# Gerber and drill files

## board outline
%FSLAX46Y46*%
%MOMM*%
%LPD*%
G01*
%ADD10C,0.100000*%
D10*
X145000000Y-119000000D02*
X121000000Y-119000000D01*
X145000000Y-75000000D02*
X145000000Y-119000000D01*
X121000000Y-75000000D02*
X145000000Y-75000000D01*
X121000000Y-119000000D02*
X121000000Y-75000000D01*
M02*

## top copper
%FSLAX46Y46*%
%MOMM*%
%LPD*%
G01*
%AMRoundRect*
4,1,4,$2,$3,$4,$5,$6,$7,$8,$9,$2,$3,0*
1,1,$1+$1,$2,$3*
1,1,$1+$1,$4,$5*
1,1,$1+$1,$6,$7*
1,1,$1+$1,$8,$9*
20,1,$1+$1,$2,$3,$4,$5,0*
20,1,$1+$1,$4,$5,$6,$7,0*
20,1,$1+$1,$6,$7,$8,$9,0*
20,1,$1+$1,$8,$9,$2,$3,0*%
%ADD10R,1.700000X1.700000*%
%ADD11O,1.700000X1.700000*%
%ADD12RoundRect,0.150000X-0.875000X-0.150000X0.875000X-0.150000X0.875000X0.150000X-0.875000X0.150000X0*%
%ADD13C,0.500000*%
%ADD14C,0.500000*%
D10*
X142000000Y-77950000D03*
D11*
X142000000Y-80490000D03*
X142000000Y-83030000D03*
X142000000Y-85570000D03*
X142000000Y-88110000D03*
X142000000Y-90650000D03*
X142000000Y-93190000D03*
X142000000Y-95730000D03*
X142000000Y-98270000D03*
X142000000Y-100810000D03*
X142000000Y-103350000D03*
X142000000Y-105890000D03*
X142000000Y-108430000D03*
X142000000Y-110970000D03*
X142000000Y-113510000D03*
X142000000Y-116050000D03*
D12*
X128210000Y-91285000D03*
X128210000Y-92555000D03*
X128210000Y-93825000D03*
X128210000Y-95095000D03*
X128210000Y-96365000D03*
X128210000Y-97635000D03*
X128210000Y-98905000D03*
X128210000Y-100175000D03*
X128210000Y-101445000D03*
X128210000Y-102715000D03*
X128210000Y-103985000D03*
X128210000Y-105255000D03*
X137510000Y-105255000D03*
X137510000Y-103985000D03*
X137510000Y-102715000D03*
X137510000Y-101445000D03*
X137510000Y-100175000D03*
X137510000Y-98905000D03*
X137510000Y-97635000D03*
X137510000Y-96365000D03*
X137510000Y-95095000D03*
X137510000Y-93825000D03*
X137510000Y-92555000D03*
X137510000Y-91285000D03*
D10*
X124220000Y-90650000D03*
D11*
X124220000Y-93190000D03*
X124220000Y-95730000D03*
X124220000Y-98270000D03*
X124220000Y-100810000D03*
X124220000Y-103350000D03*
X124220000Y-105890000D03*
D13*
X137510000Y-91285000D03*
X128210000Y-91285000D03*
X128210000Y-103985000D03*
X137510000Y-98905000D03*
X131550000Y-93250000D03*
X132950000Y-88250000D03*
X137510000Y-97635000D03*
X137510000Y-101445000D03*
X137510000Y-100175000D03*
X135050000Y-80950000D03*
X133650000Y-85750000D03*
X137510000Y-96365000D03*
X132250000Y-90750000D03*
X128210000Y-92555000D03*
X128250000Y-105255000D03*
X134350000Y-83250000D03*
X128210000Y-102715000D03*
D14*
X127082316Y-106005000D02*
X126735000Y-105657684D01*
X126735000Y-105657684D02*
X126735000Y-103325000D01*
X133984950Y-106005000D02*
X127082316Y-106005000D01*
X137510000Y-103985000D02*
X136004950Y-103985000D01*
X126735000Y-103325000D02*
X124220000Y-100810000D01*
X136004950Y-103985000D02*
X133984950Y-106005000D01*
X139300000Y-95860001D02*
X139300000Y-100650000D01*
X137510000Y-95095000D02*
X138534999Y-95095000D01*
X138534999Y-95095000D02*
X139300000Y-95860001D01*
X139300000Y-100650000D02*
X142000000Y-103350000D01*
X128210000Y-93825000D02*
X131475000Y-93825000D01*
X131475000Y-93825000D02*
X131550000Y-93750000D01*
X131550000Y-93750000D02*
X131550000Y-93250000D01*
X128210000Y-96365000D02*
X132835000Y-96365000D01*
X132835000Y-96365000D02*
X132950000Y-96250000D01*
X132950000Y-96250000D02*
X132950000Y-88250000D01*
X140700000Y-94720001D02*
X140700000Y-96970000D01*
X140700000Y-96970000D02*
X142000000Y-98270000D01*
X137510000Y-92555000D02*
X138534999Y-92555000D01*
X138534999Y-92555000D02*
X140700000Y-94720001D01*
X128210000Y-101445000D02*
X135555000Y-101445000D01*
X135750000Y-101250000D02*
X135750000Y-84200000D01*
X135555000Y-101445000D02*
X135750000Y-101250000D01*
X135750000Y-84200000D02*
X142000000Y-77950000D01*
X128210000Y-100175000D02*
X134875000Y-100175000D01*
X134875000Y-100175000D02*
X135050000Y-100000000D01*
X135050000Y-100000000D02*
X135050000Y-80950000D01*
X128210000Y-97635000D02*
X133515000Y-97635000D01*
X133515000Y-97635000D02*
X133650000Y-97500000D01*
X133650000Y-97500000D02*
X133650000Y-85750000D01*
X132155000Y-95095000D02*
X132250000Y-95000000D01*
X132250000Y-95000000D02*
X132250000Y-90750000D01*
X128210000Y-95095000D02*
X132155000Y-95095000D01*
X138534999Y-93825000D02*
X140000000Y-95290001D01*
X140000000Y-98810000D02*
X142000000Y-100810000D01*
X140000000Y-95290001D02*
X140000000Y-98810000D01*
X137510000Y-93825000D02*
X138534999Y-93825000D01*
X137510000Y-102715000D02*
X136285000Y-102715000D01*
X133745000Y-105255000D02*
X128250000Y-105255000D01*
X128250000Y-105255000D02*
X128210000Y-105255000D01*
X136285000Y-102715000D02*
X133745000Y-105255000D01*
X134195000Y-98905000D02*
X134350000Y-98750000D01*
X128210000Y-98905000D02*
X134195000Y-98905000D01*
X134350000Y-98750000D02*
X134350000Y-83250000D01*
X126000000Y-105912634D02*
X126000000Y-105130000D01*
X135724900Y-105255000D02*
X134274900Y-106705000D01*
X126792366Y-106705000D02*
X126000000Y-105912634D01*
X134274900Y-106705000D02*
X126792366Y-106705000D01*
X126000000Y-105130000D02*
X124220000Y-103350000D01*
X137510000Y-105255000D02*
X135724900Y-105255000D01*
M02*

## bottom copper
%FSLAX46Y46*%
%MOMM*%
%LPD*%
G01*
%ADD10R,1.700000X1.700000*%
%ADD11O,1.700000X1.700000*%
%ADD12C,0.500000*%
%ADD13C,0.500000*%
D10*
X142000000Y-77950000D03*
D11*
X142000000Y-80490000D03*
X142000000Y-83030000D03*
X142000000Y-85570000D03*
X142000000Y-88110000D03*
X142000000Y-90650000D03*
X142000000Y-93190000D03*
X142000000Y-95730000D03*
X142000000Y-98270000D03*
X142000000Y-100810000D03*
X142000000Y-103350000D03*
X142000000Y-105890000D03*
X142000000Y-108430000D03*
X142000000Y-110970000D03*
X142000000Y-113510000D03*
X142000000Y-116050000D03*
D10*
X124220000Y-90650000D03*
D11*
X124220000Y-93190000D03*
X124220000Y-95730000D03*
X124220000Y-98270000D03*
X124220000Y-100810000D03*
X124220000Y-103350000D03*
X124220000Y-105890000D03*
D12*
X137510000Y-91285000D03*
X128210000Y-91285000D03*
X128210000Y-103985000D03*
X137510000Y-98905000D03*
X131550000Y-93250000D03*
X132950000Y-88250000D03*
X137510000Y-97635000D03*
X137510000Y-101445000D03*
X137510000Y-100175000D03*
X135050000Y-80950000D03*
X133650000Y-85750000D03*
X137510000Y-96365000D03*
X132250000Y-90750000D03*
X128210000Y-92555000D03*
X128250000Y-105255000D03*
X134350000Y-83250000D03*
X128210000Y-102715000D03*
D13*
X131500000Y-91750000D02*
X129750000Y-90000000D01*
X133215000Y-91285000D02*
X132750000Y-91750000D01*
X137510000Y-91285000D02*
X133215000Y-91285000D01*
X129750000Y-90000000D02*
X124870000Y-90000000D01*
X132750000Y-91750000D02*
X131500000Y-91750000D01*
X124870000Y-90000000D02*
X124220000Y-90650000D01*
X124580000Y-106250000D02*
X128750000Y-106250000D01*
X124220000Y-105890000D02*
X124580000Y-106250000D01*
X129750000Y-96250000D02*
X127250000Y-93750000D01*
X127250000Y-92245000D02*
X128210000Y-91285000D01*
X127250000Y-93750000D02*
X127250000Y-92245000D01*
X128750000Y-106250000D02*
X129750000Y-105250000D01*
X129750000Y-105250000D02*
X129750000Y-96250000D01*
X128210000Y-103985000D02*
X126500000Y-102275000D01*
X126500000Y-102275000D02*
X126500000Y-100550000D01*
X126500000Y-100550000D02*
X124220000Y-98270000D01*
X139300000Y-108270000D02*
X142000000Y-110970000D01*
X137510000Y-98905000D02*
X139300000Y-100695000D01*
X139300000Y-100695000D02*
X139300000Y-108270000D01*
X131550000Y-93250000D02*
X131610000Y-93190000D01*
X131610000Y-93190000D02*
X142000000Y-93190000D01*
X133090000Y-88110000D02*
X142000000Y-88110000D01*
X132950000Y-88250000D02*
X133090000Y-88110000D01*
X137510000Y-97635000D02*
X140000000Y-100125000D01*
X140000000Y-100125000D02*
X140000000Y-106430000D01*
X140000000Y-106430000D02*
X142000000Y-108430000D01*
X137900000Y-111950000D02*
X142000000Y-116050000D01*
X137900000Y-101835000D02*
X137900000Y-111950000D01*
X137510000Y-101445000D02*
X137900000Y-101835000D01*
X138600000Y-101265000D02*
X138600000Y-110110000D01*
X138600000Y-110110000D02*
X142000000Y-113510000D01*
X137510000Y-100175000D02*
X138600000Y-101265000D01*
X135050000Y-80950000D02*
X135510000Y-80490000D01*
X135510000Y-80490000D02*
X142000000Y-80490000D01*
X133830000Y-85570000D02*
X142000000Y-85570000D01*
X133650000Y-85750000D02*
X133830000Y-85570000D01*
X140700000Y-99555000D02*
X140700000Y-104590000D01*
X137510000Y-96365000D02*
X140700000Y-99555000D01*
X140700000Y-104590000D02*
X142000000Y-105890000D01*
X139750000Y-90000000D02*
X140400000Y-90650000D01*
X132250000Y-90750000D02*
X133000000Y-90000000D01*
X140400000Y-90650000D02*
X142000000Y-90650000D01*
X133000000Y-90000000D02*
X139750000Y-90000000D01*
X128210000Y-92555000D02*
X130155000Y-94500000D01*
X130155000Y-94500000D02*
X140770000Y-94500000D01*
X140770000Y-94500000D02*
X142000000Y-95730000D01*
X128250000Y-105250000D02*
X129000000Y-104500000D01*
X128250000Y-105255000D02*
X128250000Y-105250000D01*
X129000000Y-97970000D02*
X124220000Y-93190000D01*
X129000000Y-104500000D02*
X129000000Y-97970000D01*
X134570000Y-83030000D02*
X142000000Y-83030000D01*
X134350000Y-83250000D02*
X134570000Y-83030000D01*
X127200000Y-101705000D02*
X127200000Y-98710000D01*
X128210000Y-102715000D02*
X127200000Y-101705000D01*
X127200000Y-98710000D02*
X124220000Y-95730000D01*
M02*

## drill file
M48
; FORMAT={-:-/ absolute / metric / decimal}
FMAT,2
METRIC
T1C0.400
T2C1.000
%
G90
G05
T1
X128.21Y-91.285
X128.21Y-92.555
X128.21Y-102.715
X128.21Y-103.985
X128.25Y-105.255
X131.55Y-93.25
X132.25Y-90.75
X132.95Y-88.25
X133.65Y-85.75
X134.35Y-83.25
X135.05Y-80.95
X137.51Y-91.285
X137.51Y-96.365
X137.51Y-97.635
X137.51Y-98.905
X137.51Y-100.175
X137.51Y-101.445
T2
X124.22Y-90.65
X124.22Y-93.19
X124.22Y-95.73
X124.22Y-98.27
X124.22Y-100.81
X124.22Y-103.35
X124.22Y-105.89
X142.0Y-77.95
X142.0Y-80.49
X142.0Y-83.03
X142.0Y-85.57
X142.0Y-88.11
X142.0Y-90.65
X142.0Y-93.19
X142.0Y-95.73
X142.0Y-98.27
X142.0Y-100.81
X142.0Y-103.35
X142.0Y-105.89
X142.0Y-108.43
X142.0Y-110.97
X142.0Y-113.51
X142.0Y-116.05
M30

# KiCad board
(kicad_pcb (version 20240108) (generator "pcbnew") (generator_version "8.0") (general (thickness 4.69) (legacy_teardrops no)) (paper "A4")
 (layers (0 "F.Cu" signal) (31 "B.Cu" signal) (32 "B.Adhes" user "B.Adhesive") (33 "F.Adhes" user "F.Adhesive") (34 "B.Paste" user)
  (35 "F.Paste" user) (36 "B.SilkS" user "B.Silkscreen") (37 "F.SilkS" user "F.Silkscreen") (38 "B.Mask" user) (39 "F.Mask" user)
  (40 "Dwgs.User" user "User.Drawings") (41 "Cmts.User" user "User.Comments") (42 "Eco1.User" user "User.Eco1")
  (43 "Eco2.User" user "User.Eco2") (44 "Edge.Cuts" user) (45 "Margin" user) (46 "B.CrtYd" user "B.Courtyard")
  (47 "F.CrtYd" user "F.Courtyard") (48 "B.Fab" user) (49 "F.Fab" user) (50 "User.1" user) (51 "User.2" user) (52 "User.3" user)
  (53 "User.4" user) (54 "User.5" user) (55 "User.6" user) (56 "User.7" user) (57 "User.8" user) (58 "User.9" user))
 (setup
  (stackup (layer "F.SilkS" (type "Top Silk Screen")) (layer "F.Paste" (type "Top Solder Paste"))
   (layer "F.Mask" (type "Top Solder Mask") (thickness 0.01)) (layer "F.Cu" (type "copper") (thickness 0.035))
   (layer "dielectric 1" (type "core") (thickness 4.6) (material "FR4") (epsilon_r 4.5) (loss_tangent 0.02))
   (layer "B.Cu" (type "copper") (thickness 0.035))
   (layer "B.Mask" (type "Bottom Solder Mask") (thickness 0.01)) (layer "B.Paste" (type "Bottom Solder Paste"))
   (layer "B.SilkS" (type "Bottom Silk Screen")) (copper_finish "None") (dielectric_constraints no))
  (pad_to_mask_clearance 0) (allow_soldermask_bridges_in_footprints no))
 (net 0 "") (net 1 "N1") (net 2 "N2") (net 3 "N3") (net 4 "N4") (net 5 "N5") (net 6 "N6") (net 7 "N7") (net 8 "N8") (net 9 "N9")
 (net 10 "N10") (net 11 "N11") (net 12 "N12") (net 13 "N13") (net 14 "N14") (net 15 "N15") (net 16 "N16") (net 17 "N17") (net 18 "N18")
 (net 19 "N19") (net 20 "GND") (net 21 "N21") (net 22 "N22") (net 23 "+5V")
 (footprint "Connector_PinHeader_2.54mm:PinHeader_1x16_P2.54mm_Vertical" (layer "F.Cu") (at 142 77.95)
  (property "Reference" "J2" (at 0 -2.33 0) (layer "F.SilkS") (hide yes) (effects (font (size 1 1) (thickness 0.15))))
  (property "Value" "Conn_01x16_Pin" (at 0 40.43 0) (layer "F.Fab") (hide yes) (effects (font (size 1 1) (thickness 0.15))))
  (pad "1" thru_hole rect (at 0 0) (size 1.7 1.7) (drill 1) (layers "*.Cu" "*.Mask") (remove_unused_layers no) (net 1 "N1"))
  (pad "2" thru_hole oval (at 0 2.54) (size 1.7 1.7) (drill 1) (layers "*.Cu" "*.Mask") (remove_unused_layers no) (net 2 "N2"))
  (pad "3" thru_hole oval (at 0 5.08) (size 1.7 1.7) (drill 1) (layers "*.Cu" "*.Mask") (remove_unused_layers no) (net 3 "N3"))
  (pad "4" thru_hole oval (at 0 7.62) (size 1.7 1.7) (drill 1) (layers "*.Cu" "*.Mask") (remove_unused_layers no) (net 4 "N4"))
  (pad "5" thru_hole oval (at 0 10.16) (size 1.7 1.7) (drill 1) (layers "*.Cu" "*.Mask") (remove_unused_layers no) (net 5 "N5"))
  (pad "6" thru_hole oval (at 0 12.7) (size 1.7 1.7) (drill 1) (layers "*.Cu" "*.Mask") (remove_unused_layers no) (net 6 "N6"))
  (pad "7" thru_hole oval (at 0 15.24) (size 1.7 1.7) (drill 1) (layers "*.Cu" "*.Mask") (remove_unused_layers no) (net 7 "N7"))
  (pad "8" thru_hole oval (at 0 17.78) (size 1.7 1.7) (drill 1) (layers "*.Cu" "*.Mask") (remove_unused_layers no) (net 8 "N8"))
  (pad "9" thru_hole oval (at 0 20.32) (size 1.7 1.7) (drill 1) (layers "*.Cu" "*.Mask") (remove_unused_layers no) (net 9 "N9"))
  (pad "10" thru_hole oval (at 0 22.86) (size 1.7 1.7) (drill 1) (layers "*.Cu" "*.Mask") (remove_unused_layers no) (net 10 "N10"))
  (pad "11" thru_hole oval (at 0 25.4) (size 1.7 1.7) (drill 1) (layers "*.Cu" "*.Mask") (remove_unused_layers no) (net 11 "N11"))
  (pad "12" thru_hole oval (at 0 27.94) (size 1.7 1.7) (drill 1) (layers "*.Cu" "*.Mask") (remove_unused_layers no) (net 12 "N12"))
  (pad "13" thru_hole oval (at 0 30.48) (size 1.7 1.7) (drill 1) (layers "*.Cu" "*.Mask") (remove_unused_layers no) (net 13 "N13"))
  (pad "14" thru_hole oval (at 0 33.02) (size 1.7 1.7) (drill 1) (layers "*.Cu" "*.Mask") (remove_unused_layers no) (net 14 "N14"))
  (pad "15" thru_hole oval (at 0 35.56) (size 1.7 1.7) (drill 1) (layers "*.Cu" "*.Mask") (remove_unused_layers no) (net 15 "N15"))
  (pad "16" thru_hole oval (at 0 38.1) (size 1.7 1.7) (drill 1) (layers "*.Cu" "*.Mask") (remove_unused_layers no) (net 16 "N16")))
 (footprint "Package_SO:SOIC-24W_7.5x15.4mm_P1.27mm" (layer "F.Cu") (at 132.86 98.27)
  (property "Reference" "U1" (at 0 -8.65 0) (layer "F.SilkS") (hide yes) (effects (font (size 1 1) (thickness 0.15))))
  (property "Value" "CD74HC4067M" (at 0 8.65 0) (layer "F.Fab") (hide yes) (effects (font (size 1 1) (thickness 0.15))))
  (pad "1" smd roundrect (at -4.65 -6.985) (size 2.05 0.6) (layers "F.Cu" "F.Paste" "F.Mask") (roundrect_rratio 0.25) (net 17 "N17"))
  (pad "2" smd roundrect (at -4.65 -5.715) (size 2.05 0.6) (layers "F.Cu" "F.Paste" "F.Mask") (roundrect_rratio 0.25) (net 8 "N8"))
  (pad "3" smd roundrect (at -4.65 -4.445) (size 2.05 0.6) (layers "F.Cu" "F.Paste" "F.Mask") (roundrect_rratio 0.25) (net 7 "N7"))
  (pad "4" smd roundrect (at -4.65 -3.175) (size 2.05 0.6) (layers "F.Cu" "F.Paste" "F.Mask") (roundrect_rratio 0.25) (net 6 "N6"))
  (pad "5" smd roundrect (at -4.65 -1.905) (size 2.05 0.6) (layers "F.Cu" "F.Paste" "F.Mask") (roundrect_rratio 0.25) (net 5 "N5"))
  (pad "6" smd roundrect (at -4.65 -0.635) (size 2.05 0.6) (layers "F.Cu" "F.Paste" "F.Mask") (roundrect_rratio 0.25) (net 4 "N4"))
  (pad "7" smd roundrect (at -4.65 0.635) (size 2.05 0.6) (layers "F.Cu" "F.Paste" "F.Mask") (roundrect_rratio 0.25) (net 3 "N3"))
  (pad "8" smd roundrect (at -4.65 1.905) (size 2.05 0.6) (layers "F.Cu" "F.Paste" "F.Mask") (roundrect_rratio 0.25) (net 2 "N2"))
  (pad "9" smd roundrect (at -4.65 3.175) (size 2.05 0.6) (layers "F.Cu" "F.Paste" "F.Mask") (roundrect_rratio 0.25) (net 1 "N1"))
  (pad "10" smd roundrect (at -4.65 4.445) (size 2.05 0.6) (layers "F.Cu" "F.Paste" "F.Mask") (roundrect_rratio 0.25) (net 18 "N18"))
  (pad "11" smd roundrect (at -4.65 5.715) (size 2.05 0.6) (layers "F.Cu" "F.Paste" "F.Mask") (roundrect_rratio 0.25) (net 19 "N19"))
  (pad "12" smd roundrect (at -4.65 6.985) (size 2.05 0.6) (layers "F.Cu" "F.Paste" "F.Mask") (roundrect_rratio 0.25) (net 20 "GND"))
  (pad "13" smd roundrect (at 4.65 6.985) (size 2.05 0.6) (layers "F.Cu" "F.Paste" "F.Mask") (roundrect_rratio 0.25) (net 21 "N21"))
  (pad "14" smd roundrect (at 4.65 5.715) (size 2.05 0.6) (layers "F.Cu" "F.Paste" "F.Mask") (roundrect_rratio 0.25) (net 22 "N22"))
  (pad "15" smd roundrect (at 4.65 4.445) (size 2.05 0.6) (layers "F.Cu" "F.Paste" "F.Mask") (roundrect_rratio 0.25) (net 20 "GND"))
  (pad "16" smd roundrect (at 4.65 3.175) (size 2.05 0.6) (layers "F.Cu" "F.Paste" "F.Mask") (roundrect_rratio 0.25) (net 16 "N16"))
  (pad "17" smd roundrect (at 4.65 1.905) (size 2.05 0.6) (layers "F.Cu" "F.Paste" "F.Mask") (roundrect_rratio 0.25) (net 15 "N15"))
  (pad "18" smd roundrect (at 4.65 0.635) (size 2.05 0.6) (layers "F.Cu" "F.Paste" "F.Mask") (roundrect_rratio 0.25) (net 14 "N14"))
  (pad "19" smd roundrect (at 4.65 -0.635) (size 2.05 0.6) (layers "F.Cu" "F.Paste" "F.Mask") (roundrect_rratio 0.25) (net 13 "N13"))
  (pad "20" smd roundrect (at 4.65 -1.905) (size 2.05 0.6) (layers "F.Cu" "F.Paste" "F.Mask") (roundrect_rratio 0.25) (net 12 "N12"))
  (pad "21" smd roundrect (at 4.65 -3.175) (size 2.05 0.6) (layers "F.Cu" "F.Paste" "F.Mask") (roundrect_rratio 0.25) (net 11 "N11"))
  (pad "22" smd roundrect (at 4.65 -4.445) (size 2.05 0.6) (layers "F.Cu" "F.Paste" "F.Mask") (roundrect_rratio 0.25) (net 10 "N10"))
  (pad "23" smd roundrect (at 4.65 -5.715) (size 2.05 0.6) (layers "F.Cu" "F.Paste" "F.Mask") (roundrect_rratio 0.25) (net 9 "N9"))
  (pad "24" smd roundrect (at 4.65 -6.985) (size 2.05 0.6) (layers "F.Cu" "F.Paste" "F.Mask") (roundrect_rratio 0.25) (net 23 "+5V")))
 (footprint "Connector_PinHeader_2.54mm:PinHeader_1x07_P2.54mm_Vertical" (layer "F.Cu") (at 124.22 90.65)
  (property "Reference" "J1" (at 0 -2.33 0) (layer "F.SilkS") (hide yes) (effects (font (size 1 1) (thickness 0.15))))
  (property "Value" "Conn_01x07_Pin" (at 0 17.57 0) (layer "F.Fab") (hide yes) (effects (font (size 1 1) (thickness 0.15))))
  (pad "1" thru_hole rect (at 0 0) (size 1.7 1.7) (drill 1) (layers "*.Cu" "*.Mask") (remove_unused_layers no) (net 23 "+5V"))
  (pad "2" thru_hole oval (at 0 2.54) (size 1.7 1.7) (drill 1) (layers "*.Cu" "*.Mask") (remove_unused_layers no) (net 20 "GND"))
  (pad "3" thru_hole oval (at 0 5.08) (size 1.7 1.7) (drill 1) (layers "*.Cu" "*.Mask") (remove_unused_layers no) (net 18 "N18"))
  (pad "4" thru_hole oval (at 0 7.62) (size 1.7 1.7) (drill 1) (layers "*.Cu" "*.Mask") (remove_unused_layers no) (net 19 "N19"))
  (pad "5" thru_hole oval (at 0 10.16) (size 1.7 1.7) (drill 1) (layers "*.Cu" "*.Mask") (remove_unused_layers no) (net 22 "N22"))
  (pad "6" thru_hole oval (at 0 12.7) (size 1.7 1.7) (drill 1) (layers "*.Cu" "*.Mask") (remove_unused_layers no) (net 21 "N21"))
  (pad "7" thru_hole oval (at 0 15.24) (size 1.7 1.7) (drill 1) (layers "*.Cu" "*.Mask") (remove_unused_layers no) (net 17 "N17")))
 (gr_line (start 145 119) (end 121 119) (stroke (width 0.1) (type default)) (layer "Edge.Cuts"))
 (gr_line (start 145 75) (end 145 119) (stroke (width 0.1) (type default)) (layer "Edge.Cuts"))
 (gr_line (start 121 75) (end 145 75) (stroke (width 0.1) (type default)) (layer "Edge.Cuts"))
 (gr_line (start 121 119) (end 121 75) (stroke (width 0.1) (type default)) (layer "Edge.Cuts"))
 (via (at 137.51 91.285) (size 0.5) (drill 0.4) (layers "F.Cu" "B.Cu") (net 23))
 (segment (start 131.5 91.75) (end 129.75 90) (width 0.5) (layer "B.Cu") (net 23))
 (segment (start 133.215 91.285) (end 132.75 91.75) (width 0.5) (layer "B.Cu") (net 23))
 (segment (start 137.51 91.285) (end 133.215 91.285) (width 0.5) (layer "B.Cu") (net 23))
 (segment (start 129.75 90) (end 124.87 90) (width 0.5) (layer "B.Cu") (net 23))
 (segment (start 132.75 91.75) (end 131.5 91.75) (width 0.5) (layer "B.Cu") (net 23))
 (segment (start 124.87 90) (end 124.22 90.65) (width 0.5) (layer "B.Cu") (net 23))
 (via (at 128.21 91.285) (size 0.5) (drill 0.4) (layers "F.Cu" "B.Cu") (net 17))
 (segment (start 124.58 106.25) (end 128.75 106.25) (width 0.5) (layer "B.Cu") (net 17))
 (segment (start 124.22 105.89) (end 124.58 106.25) (width 0.5) (layer "B.Cu") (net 17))
 (segment (start 129.75 96.25) (end 127.25 93.75) (width 0.5) (layer "B.Cu") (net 17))
 (segment (start 127.25 92.245) (end 128.21 91.285) (width 0.5) (layer "B.Cu") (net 17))
 (segment (start 127.25 93.75) (end 127.25 92.245) (width 0.5) (layer "B.Cu") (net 17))
 (segment (start 128.75 106.25) (end 129.75 105.25) (width 0.5) (layer "B.Cu") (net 17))
 (segment (start 129.75 105.25) (end 129.75 96.25) (width 0.5) (layer "B.Cu") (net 17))
 (segment (start 127.082316 106.005) (end 126.735 105.657684) (width 0.5) (layer "F.Cu") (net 22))
 (segment (start 126.735 105.657684) (end 126.735 103.325) (width 0.5) (layer "F.Cu") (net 22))
 (segment (start 133.98495 106.005) (end 127.082316 106.005) (width 0.5) (layer "F.Cu") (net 22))
 (segment (start 137.51 103.985) (end 136.00495 103.985) (width 0.5) (layer "F.Cu") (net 22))
 (segment (start 126.735 103.325) (end 124.22 100.81) (width 0.5) (layer "F.Cu") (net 22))
 (segment (start 136.00495 103.985) (end 133.98495 106.005) (width 0.5) (layer "F.Cu") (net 22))
 (via (at 128.21 103.985) (size 0.5) (drill 0.4) (layers "F.Cu" "B.Cu") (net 19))
 (segment (start 128.21 103.985) (end 126.5 102.275) (width 0.5) (layer "B.Cu") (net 19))
 (segment (start 126.5 102.275) (end 126.5 100.55) (width 0.5) (layer "B.Cu") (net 19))
 (segment (start 126.5 100.55) (end 124.22 98.27) (width 0.5) (layer "B.Cu") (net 19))
 (via (at 137.51 98.905) (size 0.5) (drill 0.4) (layers "F.Cu" "B.Cu") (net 14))
 (segment (start 139.3 108.27) (end 142 110.97) (width 0.5) (layer "B.Cu") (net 14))
 (segment (start 137.51 98.905) (end 139.3 100.695) (width 0.5) (layer "B.Cu") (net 14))
 (segment (start 139.3 100.695) (end 139.3 108.27) (width 0.5) (layer "B.Cu") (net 14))
 (segment (start 139.3 95.860001) (end 139.3 100.65) (width 0.5) (layer "F.Cu") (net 11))
 (segment (start 137.51 95.095) (end 138.534999 95.095) (width 0.5) (layer "F.Cu") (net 11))
 (segment (start 138.534999 95.095) (end 139.3 95.860001) (width 0.5) (layer "F.Cu") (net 11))
 (segment (start 139.3 100.65) (end 142 103.35) (width 0.5) (layer "F.Cu") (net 11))
 (segment (start 128.21 93.825) (end 131.475 93.825) (width 0.5) (layer "F.Cu") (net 7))
 (segment (start 131.475 93.825) (end 131.55 93.75) (width 0.5) (layer "F.Cu") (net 7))
 (segment (start 131.55 93.75) (end 131.55 93.25) (width 0.5) (layer "F.Cu") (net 7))
 (via (at 131.55 93.25) (size 0.5) (drill 0.4) (layers "F.Cu" "B.Cu") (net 7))
 (segment (start 131.55 93.25) (end 131.61 93.19) (width 0.5) (layer "B.Cu") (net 7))
 (segment (start 131.61 93.19) (end 142 93.19) (width 0.5) (layer "B.Cu") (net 7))
 (segment (start 128.21 96.365) (end 132.835 96.365) (width 0.5) (layer "F.Cu") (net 5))
 (segment (start 132.835 96.365) (end 132.95 96.25) (width 0.5) (layer "F.Cu") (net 5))
 (segment (start 132.95 96.25) (end 132.95 88.25) (width 0.5) (layer "F.Cu") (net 5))
 (via (at 132.95 88.25) (size 0.5) (drill 0.4) (layers "F.Cu" "B.Cu") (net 5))
 (segment (start 133.09 88.11) (end 142 88.11) (width 0.5) (layer "B.Cu") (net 5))
 (segment (start 132.95 88.25) (end 133.09 88.11) (width 0.5) (layer "B.Cu") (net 5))
 (via (at 137.51 97.635) (size 0.5) (drill 0.4) (layers "F.Cu" "B.Cu") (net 13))
 (segment (start 137.51 97.635) (end 140 100.125) (width 0.5) (layer "B.Cu") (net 13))
 (segment (start 140 100.125) (end 140 106.43) (width 0.5) (layer "B.Cu") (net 13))
 (segment (start 140 106.43) (end 142 108.43) (width 0.5) (layer "B.Cu") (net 13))
 (segment (start 140.7 94.720001) (end 140.7 96.97) (width 0.5) (layer "F.Cu") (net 9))
 (segment (start 140.7 96.97) (end 142 98.27) (width 0.5) (layer "F.Cu") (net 9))
 (segment (start 137.51 92.555) (end 138.534999 92.555) (width 0.5) (layer "F.Cu") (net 9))
 (segment (start 138.534999 92.555) (end 140.7 94.720001) (width 0.5) (layer "F.Cu") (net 9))
 (via (at 137.51 101.445) (size 0.5) (drill 0.4) (layers "F.Cu" "B.Cu") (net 16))
 (segment (start 137.9 111.95) (end 142 116.05) (width 0.5) (layer "B.Cu") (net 16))
 (segment (start 137.9 101.835) (end 137.9 111.95) (width 0.5) (layer "B.Cu") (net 16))
 (segment (start 137.51 101.445) (end 137.9 101.835) (width 0.5) (layer "B.Cu") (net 16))
 (via (at 137.51 100.175) (size 0.5) (drill 0.4) (layers "F.Cu" "B.Cu") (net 15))
 (segment (start 138.6 101.265) (end 138.6 110.11) (width 0.5) (layer "B.Cu") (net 15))
 (segment (start 138.6 110.11) (end 142 113.51) (width 0.5) (layer "B.Cu") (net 15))
 (segment (start 137.51 100.175) (end 138.6 101.265) (width 0.5) (layer "B.Cu") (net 15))
 (segment (start 128.21 101.445) (end 135.555 101.445) (width 0.5) (layer "F.Cu") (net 1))
 (segment (start 135.75 101.25) (end 135.75 84.2) (width 0.5) (layer "F.Cu") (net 1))
 (segment (start 135.555 101.445) (end 135.75 101.25) (width 0.5) (layer "F.Cu") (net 1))
 (segment (start 135.75 84.2) (end 142 77.95) (width 0.5) (layer "F.Cu") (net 1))
 (segment (start 128.21 100.175) (end 134.875 100.175) (width 0.5) (layer "F.Cu") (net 2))
 (segment (start 134.875 100.175) (end 135.05 100) (width 0.5) (layer "F.Cu") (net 2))
 (segment (start 135.05 100) (end 135.05 80.95) (width 0.5) (layer "F.Cu") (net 2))
 (via (at 135.05 80.95) (size 0.5) (drill 0.4) (layers "F.Cu" "B.Cu") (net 2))
 (segment (start 135.05 80.95) (end 135.51 80.49) (width 0.5) (layer "B.Cu") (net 2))
 (segment (start 135.51 80.49) (end 142 80.49) (width 0.5) (layer "B.Cu") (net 2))
 (segment (start 128.21 97.635) (end 133.515 97.635) (width 0.5) (layer "F.Cu") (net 4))
 (segment (start 133.515 97.635) (end 133.65 97.5) (width 0.5) (layer "F.Cu") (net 4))
 (segment (start 133.65 97.5) (end 133.65 85.75) (width 0.5) (layer "F.Cu") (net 4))
 (via (at 133.65 85.75) (size 0.5) (drill 0.4) (layers "F.Cu" "B.Cu") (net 4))
 (segment (start 133.83 85.57) (end 142 85.57) (width 0.5) (layer "B.Cu") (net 4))
 (segment (start 133.65 85.75) (end 133.83 85.57) (width 0.5) (layer "B.Cu") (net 4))
 (via (at 137.51 96.365) (size 0.5) (drill 0.4) (layers "F.Cu" "B.Cu") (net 12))
 (segment (start 140.7 99.555) (end 140.7 104.59) (width 0.5) (layer "B.Cu") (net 12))
 (segment (start 137.51 96.365) (end 140.7 99.555) (width 0.5) (layer "B.Cu") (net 12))
 (segment (start 140.7 104.59) (end 142 105.89) (width 0.5) (layer "B.Cu") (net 12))
 (segment (start 132.155 95.095) (end 132.25 95) (width 0.5) (layer "F.Cu") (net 6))
 (segment (start 132.25 95) (end 132.25 90.75) (width 0.5) (layer "F.Cu") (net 6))
 (segment (start 128.21 95.095) (end 132.155 95.095) (width 0.5) (layer "F.Cu") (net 6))
 (via (at 132.25 90.75) (size 0.5) (drill 0.4) (layers "F.Cu" "B.Cu") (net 6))
 (segment (start 139.75 90) (end 140.4 90.65) (width 0.5) (layer "B.Cu") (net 6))
 (segment (start 132.25 90.75) (end 133 90) (width 0.5) (layer "B.Cu") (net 6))
 (segment (start 140.4 90.65) (end 142 90.65) (width 0.5) (layer "B.Cu") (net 6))
 (segment (start 133 90) (end 139.75 90) (width 0.5) (layer "B.Cu") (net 6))
 (segment (start 138.534999 93.825) (end 140 95.290001) (width 0.5) (layer "F.Cu") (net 10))
 (segment (start 140 98.81) (end 142 100.81) (width 0.5) (layer "F.Cu") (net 10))
 (segment (start 140 95.290001) (end 140 98.81) (width 0.5) (layer "F.Cu") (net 10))
 (segment (start 137.51 93.825) (end 138.534999 93.825) (width 0.5) (layer "F.Cu") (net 10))
 (via (at 128.21 92.555) (size 0.5) (drill 0.4) (layers "F.Cu" "B.Cu") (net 8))
 (segment (start 128.21 92.555) (end 130.155 94.5) (width 0.5) (layer "B.Cu") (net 8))
 (segment (start 130.155 94.5) (end 140.77 94.5) (width 0.5) (layer "B.Cu") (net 8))
 (segment (start 140.77 94.5) (end 142 95.73) (width 0.5) (layer "B.Cu") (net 8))
 (segment (start 137.51 102.715) (end 136.285 102.715) (width 0.5) (layer "F.Cu") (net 20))
 (segment (start 133.745 105.255) (end 128.25 105.255) (width 0.5) (layer "F.Cu") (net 20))
 (segment (start 128.25 105.255) (end 128.21 105.255) (width 0.5) (layer "F.Cu") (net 20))
 (segment (start 136.285 102.715) (end 133.745 105.255) (width 0.5) (layer "F.Cu") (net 20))
 (via (at 128.25 105.255) (size 0.5) (drill 0.4) (layers "F.Cu" "B.Cu") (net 20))
 (segment (start 128.25 105.25) (end 129 104.5) (width 0.5) (layer "B.Cu") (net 20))
 (segment (start 128.25 105.255) (end 128.25 105.25) (width 0.5) (layer "B.Cu") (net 20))
 (segment (start 129 97.97) (end 124.22 93.19) (width 0.5) (layer "B.Cu") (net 20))
 (segment (start 129 104.5) (end 129 97.97) (width 0.5) (layer "B.Cu") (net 20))
 (segment (start 134.195 98.905) (end 134.35 98.75) (width 0.5) (layer "F.Cu") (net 3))
 (segment (start 128.21 98.905) (end 134.195 98.905) (width 0.5) (layer "F.Cu") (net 3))
 (segment (start 134.35 98.75) (end 134.35 83.25) (width 0.5) (layer "F.Cu") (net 3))
 (via (at 134.35 83.25) (size 0.5) (drill 0.4) (layers "F.Cu" "B.Cu") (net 3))
 (segment (start 134.57 83.03) (end 142 83.03) (width 0.5) (layer "B.Cu") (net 3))
 (segment (start 134.35 83.25) (end 134.57 83.03) (width 0.5) (layer "B.Cu") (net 3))
 (via (at 128.21 102.715) (size 0.5) (drill 0.4) (layers "F.Cu" "B.Cu") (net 18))
 (segment (start 127.2 101.705) (end 127.2 98.71) (width 0.5) (layer "B.Cu") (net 18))
 (segment (start 128.21 102.715) (end 127.2 101.705) (width 0.5) (layer "B.Cu") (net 18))
 (segment (start 127.2 98.71) (end 124.22 95.73) (width 0.5) (layer "B.Cu") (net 18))
 (segment (start 126 105.912634) (end 126 105.13) (width 0.5) (layer "F.Cu") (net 21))
 (segment (start 135.7249 105.255) (end 134.2749 106.705) (width 0.5) (layer "F.Cu") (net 21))
 (segment (start 126.792366 106.705) (end 126 105.912634) (width 0.5) (layer "F.Cu") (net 21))
 (segment (start 134.2749 106.705) (end 126.792366 106.705) (width 0.5) (layer "F.Cu") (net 21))
 (segment (start 126 105.13) (end 124.22 103.35) (width 0.5) (layer "F.Cu") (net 21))
 (segment (start 137.51 105.255) (end 135.7249 105.255) (width 0.5) (layer "F.Cu") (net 21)))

